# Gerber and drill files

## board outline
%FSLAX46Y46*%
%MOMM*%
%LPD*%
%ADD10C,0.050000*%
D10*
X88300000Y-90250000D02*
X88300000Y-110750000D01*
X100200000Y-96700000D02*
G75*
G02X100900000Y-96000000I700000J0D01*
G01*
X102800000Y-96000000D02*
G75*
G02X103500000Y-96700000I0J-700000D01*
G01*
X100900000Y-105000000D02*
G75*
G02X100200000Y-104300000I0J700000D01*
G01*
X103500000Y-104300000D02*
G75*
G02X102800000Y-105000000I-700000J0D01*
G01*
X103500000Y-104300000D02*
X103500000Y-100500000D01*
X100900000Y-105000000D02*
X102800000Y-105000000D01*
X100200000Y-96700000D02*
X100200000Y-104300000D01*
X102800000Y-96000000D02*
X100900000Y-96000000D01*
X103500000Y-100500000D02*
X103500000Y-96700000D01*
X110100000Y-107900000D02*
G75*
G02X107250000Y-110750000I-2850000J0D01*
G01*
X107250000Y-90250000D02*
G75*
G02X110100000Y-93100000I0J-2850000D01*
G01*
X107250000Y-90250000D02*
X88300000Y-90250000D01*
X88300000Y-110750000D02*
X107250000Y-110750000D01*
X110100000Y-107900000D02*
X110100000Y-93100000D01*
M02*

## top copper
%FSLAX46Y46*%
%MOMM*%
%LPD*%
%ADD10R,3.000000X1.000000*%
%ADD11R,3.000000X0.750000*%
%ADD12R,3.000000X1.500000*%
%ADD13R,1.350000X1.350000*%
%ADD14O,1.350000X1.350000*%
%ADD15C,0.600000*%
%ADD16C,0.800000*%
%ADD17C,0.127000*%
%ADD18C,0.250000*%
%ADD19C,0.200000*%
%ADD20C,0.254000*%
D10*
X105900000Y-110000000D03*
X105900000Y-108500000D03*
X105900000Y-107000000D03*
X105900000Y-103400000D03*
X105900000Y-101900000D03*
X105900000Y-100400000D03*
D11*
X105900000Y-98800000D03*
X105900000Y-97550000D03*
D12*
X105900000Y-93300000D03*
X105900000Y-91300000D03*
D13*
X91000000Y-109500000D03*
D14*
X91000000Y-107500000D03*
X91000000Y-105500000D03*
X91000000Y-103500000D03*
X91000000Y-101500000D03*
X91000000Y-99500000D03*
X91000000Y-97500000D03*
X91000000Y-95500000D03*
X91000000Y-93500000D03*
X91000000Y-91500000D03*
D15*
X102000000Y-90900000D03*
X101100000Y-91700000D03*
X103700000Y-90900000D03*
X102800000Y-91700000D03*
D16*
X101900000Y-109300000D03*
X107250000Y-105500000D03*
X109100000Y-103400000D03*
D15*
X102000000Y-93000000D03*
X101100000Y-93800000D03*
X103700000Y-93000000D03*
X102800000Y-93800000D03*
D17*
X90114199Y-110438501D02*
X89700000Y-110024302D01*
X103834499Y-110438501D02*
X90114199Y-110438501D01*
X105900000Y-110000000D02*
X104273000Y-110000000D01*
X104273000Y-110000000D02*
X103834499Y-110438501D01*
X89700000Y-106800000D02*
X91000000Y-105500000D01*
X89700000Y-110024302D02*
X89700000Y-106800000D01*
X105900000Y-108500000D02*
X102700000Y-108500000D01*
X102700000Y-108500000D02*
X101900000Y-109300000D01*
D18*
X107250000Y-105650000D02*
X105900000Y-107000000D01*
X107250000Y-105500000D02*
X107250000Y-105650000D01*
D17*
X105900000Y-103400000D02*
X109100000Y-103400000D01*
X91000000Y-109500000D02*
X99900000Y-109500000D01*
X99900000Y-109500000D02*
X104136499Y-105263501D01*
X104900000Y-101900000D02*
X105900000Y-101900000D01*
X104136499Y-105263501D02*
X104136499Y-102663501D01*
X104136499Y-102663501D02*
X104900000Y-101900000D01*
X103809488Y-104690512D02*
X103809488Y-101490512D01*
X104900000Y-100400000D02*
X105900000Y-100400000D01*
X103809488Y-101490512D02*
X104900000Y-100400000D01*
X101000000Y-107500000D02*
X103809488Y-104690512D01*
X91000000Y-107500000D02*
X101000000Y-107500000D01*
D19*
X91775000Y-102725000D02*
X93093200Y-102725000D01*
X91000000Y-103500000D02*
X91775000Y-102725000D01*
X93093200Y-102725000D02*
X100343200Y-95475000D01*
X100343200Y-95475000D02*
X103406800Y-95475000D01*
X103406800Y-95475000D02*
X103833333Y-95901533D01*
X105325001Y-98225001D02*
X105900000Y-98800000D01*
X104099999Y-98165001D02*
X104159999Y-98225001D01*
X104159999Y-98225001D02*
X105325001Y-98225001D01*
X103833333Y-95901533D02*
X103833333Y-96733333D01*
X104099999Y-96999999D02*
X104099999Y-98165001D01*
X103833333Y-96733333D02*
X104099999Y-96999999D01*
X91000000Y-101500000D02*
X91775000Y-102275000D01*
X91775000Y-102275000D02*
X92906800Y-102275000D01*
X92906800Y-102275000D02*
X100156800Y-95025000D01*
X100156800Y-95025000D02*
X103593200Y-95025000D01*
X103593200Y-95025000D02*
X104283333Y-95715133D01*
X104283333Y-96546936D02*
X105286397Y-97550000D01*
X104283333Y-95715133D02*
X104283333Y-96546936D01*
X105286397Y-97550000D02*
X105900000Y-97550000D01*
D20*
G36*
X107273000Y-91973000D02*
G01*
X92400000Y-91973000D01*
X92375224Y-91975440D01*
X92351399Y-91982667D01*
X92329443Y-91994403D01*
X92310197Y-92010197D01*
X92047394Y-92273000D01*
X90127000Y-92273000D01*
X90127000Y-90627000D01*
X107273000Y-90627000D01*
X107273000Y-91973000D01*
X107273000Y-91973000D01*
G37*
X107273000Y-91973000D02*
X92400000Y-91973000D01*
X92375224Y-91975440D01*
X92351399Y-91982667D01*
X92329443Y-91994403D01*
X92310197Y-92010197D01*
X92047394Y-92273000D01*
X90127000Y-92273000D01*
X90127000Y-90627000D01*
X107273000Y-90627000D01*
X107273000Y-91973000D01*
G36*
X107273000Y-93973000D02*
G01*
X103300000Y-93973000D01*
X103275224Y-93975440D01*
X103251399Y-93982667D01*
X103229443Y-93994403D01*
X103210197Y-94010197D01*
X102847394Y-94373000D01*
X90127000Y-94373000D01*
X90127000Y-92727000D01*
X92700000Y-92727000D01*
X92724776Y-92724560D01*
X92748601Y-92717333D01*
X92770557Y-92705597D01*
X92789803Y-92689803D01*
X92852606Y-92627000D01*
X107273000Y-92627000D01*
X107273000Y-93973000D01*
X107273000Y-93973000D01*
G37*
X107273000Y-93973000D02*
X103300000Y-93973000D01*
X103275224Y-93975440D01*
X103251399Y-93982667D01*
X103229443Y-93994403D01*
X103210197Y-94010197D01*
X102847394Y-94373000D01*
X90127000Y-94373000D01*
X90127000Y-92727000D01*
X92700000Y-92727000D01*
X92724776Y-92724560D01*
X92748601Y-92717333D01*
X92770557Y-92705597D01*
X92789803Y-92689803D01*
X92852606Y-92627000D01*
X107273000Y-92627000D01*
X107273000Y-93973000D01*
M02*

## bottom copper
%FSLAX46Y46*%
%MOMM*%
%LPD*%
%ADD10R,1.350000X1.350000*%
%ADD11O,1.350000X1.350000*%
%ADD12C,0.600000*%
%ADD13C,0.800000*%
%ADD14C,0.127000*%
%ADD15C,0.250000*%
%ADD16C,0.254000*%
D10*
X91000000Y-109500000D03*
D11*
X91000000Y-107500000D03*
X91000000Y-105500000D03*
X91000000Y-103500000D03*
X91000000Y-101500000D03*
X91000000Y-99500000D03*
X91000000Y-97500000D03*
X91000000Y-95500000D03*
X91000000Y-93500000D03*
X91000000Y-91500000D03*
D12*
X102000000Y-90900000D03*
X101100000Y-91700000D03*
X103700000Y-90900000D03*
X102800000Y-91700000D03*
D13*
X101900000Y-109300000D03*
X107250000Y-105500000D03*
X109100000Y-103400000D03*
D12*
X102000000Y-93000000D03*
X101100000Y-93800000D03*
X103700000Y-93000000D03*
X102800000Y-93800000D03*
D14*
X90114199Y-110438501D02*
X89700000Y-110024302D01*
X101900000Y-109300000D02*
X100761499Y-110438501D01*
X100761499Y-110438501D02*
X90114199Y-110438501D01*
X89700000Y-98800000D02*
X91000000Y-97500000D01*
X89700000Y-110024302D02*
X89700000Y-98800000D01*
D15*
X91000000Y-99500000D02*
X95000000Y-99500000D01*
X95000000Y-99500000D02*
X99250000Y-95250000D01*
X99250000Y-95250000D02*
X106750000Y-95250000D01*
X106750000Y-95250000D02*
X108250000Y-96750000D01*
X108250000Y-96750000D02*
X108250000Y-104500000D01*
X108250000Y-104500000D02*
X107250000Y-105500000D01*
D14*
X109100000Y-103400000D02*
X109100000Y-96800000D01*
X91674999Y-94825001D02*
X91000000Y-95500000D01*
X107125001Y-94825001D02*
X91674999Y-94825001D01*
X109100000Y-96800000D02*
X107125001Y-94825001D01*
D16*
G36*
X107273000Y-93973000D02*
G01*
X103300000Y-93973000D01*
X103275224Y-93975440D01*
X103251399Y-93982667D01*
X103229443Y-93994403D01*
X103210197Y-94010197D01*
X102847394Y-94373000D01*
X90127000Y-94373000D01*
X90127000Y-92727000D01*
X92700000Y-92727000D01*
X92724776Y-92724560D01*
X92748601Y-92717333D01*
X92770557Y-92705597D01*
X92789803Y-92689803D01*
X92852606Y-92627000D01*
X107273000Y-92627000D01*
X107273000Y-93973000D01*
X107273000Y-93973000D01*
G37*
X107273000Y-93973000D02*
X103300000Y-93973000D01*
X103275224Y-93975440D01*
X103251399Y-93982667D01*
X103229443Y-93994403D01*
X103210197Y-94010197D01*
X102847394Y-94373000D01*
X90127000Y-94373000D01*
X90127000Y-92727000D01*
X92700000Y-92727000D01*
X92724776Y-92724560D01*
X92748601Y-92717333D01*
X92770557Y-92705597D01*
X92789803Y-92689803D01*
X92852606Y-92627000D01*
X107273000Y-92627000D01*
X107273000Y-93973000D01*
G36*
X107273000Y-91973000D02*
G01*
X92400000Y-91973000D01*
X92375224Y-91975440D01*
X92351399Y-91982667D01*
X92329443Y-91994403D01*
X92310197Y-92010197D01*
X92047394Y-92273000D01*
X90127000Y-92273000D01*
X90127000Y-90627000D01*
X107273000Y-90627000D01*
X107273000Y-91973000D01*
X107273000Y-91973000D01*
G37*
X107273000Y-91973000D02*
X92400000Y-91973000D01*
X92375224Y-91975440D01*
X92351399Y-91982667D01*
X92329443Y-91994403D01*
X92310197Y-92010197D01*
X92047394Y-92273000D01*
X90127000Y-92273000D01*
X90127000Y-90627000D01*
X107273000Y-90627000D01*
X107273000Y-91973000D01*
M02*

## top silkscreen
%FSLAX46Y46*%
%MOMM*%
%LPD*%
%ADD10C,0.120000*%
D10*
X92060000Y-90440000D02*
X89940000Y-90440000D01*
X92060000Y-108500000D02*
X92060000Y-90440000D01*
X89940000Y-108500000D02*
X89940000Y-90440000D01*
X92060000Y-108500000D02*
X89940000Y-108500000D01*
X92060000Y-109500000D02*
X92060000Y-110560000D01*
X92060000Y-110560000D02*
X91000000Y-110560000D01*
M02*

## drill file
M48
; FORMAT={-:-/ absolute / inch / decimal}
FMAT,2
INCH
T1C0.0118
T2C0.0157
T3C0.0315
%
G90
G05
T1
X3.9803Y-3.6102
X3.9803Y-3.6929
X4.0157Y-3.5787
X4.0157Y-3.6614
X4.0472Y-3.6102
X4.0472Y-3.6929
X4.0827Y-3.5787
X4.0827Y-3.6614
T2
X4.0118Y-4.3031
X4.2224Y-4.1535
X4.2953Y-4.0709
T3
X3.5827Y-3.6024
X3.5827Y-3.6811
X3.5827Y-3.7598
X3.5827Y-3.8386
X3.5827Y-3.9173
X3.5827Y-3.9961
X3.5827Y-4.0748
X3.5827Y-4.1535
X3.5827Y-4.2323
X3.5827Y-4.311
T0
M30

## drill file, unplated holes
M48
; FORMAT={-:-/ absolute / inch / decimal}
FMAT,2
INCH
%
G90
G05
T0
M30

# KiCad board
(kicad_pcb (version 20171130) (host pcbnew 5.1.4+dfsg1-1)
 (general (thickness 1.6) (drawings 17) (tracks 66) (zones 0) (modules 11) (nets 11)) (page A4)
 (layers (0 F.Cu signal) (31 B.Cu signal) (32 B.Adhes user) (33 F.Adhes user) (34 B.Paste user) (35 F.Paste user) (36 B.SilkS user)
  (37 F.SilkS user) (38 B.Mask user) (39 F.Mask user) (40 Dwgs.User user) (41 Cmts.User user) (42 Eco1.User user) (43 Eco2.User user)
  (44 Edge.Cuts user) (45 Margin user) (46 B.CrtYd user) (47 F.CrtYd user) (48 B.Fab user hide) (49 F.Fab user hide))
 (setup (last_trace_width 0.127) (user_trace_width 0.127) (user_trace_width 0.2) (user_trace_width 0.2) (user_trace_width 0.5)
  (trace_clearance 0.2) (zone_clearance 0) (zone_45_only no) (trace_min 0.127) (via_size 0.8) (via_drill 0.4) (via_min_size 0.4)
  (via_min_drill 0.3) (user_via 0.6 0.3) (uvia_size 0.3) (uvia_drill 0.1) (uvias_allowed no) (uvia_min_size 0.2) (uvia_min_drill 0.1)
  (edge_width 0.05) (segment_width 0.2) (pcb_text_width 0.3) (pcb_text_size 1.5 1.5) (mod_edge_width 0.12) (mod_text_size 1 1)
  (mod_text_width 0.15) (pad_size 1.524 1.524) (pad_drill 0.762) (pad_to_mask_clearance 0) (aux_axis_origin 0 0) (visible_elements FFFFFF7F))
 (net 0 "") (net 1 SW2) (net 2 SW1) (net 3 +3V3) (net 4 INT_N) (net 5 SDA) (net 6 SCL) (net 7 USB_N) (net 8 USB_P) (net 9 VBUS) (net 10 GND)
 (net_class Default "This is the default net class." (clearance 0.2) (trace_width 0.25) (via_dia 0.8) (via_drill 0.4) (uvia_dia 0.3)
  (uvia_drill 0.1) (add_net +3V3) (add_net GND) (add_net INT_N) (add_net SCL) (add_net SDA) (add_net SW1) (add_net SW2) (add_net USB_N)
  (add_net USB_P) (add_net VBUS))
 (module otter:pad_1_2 (layer F.Cu) (at 105.9 110 90)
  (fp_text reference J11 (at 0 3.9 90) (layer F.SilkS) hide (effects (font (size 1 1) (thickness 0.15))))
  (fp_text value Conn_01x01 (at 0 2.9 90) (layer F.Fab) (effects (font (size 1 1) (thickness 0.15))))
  (pad 1 smd rect (at 0 0 90) (size 1 3) (layers F.Cu F.Paste F.Mask) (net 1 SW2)))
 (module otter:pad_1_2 (layer F.Cu) (at 105.9 108.5 90)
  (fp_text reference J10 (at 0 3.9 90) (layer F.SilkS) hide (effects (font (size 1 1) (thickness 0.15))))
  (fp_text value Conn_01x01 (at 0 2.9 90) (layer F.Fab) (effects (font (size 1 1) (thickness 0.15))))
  (pad 1 smd rect (at 0 0 90) (size 1 3) (layers F.Cu F.Paste F.Mask) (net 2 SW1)))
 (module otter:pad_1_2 (layer F.Cu) (at 105.9 107 90)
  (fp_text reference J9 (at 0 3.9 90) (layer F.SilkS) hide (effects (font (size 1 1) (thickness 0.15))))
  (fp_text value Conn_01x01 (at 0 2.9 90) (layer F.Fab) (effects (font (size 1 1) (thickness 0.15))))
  (pad 1 smd rect (at 0 0 90) (size 1 3) (layers F.Cu F.Paste F.Mask) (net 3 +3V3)))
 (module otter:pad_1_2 (layer F.Cu) (at 105.9 103.4 90)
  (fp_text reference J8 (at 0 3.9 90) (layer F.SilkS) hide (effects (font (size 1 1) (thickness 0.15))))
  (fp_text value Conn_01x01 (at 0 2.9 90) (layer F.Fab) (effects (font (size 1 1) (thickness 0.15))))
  (pad 1 smd rect (at 0 0 90) (size 1 3) (layers F.Cu F.Paste F.Mask) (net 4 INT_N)))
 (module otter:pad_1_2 (layer F.Cu) (at 105.9 101.9 90)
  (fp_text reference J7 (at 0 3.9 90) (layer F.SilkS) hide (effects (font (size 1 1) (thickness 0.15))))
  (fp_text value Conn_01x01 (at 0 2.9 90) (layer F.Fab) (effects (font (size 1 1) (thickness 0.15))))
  (pad 1 smd rect (at 0 0 90) (size 1 3) (layers F.Cu F.Paste F.Mask) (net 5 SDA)))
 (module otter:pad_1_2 (layer F.Cu) (at 105.9 100.4 90)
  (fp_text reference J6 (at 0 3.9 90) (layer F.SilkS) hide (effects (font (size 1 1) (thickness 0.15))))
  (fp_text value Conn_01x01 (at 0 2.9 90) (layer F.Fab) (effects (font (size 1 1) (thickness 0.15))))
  (pad 1 smd rect (at 0 0 90) (size 1 3) (layers F.Cu F.Paste F.Mask) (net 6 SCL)))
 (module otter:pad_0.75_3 (layer F.Cu) (at 105.9 98.8 90)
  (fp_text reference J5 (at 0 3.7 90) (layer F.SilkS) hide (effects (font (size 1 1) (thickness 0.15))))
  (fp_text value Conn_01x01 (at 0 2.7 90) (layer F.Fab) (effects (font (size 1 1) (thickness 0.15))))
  (pad 1 smd rect (at 0 0 90) (size 0.75 3) (layers F.Cu F.Paste F.Mask) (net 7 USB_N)))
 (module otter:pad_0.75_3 (layer F.Cu) (at 105.9 97.55 90)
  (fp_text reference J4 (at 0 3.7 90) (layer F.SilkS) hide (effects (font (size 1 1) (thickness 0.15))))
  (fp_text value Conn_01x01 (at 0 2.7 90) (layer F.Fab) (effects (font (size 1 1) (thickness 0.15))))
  (pad 1 smd rect (at 0 0 90) (size 0.75 3) (layers F.Cu F.Paste F.Mask) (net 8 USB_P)))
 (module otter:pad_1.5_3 (layer F.Cu) (at 105.9 93.3 90)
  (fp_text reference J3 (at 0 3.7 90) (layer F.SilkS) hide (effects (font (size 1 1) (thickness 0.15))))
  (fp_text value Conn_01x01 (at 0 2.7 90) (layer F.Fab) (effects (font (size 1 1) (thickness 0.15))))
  (pad 1 smd rect (at 0 0 90) (size 1.5 3) (layers F.Cu F.Paste F.Mask) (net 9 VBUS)))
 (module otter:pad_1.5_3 (layer F.Cu) (at 105.9 91.3 90)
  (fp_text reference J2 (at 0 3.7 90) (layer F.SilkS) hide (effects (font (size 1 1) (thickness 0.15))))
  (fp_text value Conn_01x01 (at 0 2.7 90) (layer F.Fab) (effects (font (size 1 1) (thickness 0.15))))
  (pad 1 smd rect (at 0 0 90) (size 1.5 3) (layers F.Cu F.Paste F.Mask) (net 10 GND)))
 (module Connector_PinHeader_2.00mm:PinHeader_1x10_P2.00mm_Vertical (layer F.Cu) (at 91 100.5 180)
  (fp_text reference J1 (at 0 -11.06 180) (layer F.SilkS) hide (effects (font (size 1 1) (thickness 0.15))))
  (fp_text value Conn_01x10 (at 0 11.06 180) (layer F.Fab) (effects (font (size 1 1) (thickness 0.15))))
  (fp_line (start -1.06 10.06) (end 1.06 10.06) (layer F.SilkS) (width 0.12))
  (fp_line (start -1.06 -8) (end -1.06 10.06) (layer F.SilkS) (width 0.12))
  (fp_line (start 1.06 -8) (end 1.06 10.06) (layer F.SilkS) (width 0.12))
  (fp_line (start -1.06 -8) (end 1.06 -8) (layer F.SilkS) (width 0.12))
  (fp_line (start -1.06 -9) (end -1.06 -10.06) (layer F.SilkS) (width 0.12))
  (fp_line (start -1.06 -10.06) (end 0 -10.06) (layer F.SilkS) (width 0.12))
  (pad 1 thru_hole rect (at 0 -9 180) (size 1.35 1.35) (drill 0.8) (layers *.Cu *.Mask) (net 5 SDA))
  (pad 2 thru_hole oval (at 0 -7 180) (size 1.35 1.35) (drill 0.8) (layers *.Cu *.Mask) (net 6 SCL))
  (pad 3 thru_hole oval (at 0 -5 180) (size 1.35 1.35) (drill 0.8) (layers *.Cu *.Mask) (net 1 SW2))
  (pad 4 thru_hole oval (at 0 -3 180) (size 1.35 1.35) (drill 0.8) (layers *.Cu *.Mask) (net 7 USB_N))
  (pad 5 thru_hole oval (at 0 -1 180) (size 1.35 1.35) (drill 0.8) (layers *.Cu *.Mask) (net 8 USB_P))
  (pad 6 thru_hole oval (at 0 1 180) (size 1.35 1.35) (drill 0.8) (layers *.Cu *.Mask) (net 3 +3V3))
  (pad 7 thru_hole oval (at 0 3 180) (size 1.35 1.35) (drill 0.8) (layers *.Cu *.Mask) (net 2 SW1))
  (pad 8 thru_hole oval (at 0 5 180) (size 1.35 1.35) (drill 0.8) (layers *.Cu *.Mask) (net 4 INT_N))
  (pad 9 thru_hole oval (at 0 7 180) (size 1.35 1.35) (drill 0.8) (layers *.Cu *.Mask) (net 9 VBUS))
  (pad 10 thru_hole oval (at 0 9 180) (size 1.35 1.35) (drill 0.8) (layers *.Cu *.Mask) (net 10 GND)))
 (gr_line (start 88.3 90.25) (end 88.3 110.75) (layer Edge.Cuts) (width 0.05))
 (gr_arc (start 100.9 96.7) (end 100.9 96) (angle -90) (layer Edge.Cuts) (width 0.05))
 (gr_arc (start 102.8 96.7) (end 103.5 96.7) (angle -90) (layer Edge.Cuts) (width 0.05))
 (gr_arc (start 100.9 104.3) (end 100.2 104.3) (angle -90) (layer Edge.Cuts) (width 0.05))
 (gr_arc (start 102.8 104.3) (end 102.8 105) (angle -90) (layer Edge.Cuts) (width 0.05))
 (gr_line (start 103.5 104.3) (end 103.5 100.5) (layer Edge.Cuts) (width 0.05))
 (gr_line (start 100.9 105) (end 102.8 105) (layer Edge.Cuts) (width 0.05))
 (gr_line (start 100.2 96.7) (end 100.2 104.3) (layer Edge.Cuts) (width 0.05))
 (gr_line (start 102.8 96) (end 100.9 96) (layer Edge.Cuts) (width 0.05))
 (gr_line (start 103.5 100.5) (end 103.5 96.7) (layer Edge.Cuts) (width 0.05))
 (gr_arc (start 107.25 107.9) (end 107.25 110.75) (angle -90) (layer Edge.Cuts) (width 0.05))
 (gr_arc (start 107.25 93.1) (end 110.1 93.1) (angle -90) (layer Edge.Cuts) (width 0.05))
 (gr_line (start 107.25 90.25) (end 88.3 90.25) (layer Edge.Cuts) (width 0.05))
 (gr_line (start 88.3 110.75) (end 107.25 110.75) (layer Edge.Cuts) (width 0.05))
 (gr_line (start 110.1 107.9) (end 110.1 93.1) (layer Edge.Cuts) (width 0.05))
 (via (at 102 90.9) (size 0.6) (drill 0.3) (layers F.Cu B.Cu) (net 10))
 (via (at 101.1 91.7) (size 0.6) (drill 0.3) (layers F.Cu B.Cu) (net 10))
 (via (at 103.7 90.9) (size 0.6) (drill 0.3) (layers F.Cu B.Cu) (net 10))
 (via (at 102.8 91.7) (size 0.6) (drill 0.3) (layers F.Cu B.Cu) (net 10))
 (segment (start 90.114199 110.438501) (end 89.7 110.024302) (width 0.127) (layer F.Cu) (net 1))
 (segment (start 103.834499 110.438501) (end 90.114199 110.438501) (width 0.127) (layer F.Cu) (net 1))
 (segment (start 105.9 110) (end 104.273 110) (width 0.127) (layer F.Cu) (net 1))
 (segment (start 104.273 110) (end 103.834499 110.438501) (width 0.127) (layer F.Cu) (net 1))
 (segment (start 89.7 106.8) (end 91 105.5) (width 0.127) (layer F.Cu) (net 1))
 (segment (start 89.7 110.024302) (end 89.7 106.8) (width 0.127) (layer F.Cu) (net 1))
 (via (at 101.9 109.3) (size 0.8) (drill 0.4) (layers F.Cu B.Cu) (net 2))
 (segment (start 105.9 108.5) (end 102.7 108.5) (width 0.127) (layer F.Cu) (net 2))
 (segment (start 102.7 108.5) (end 101.9 109.3) (width 0.127) (layer F.Cu) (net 2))
 (segment (start 90.114199 110.438501) (end 89.7 110.024302) (width 0.127) (layer B.Cu) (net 2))
 (segment (start 101.9 109.3) (end 100.761499 110.438501) (width 0.127) (layer B.Cu) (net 2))
 (segment (start 100.761499 110.438501) (end 90.114199 110.438501) (width 0.127) (layer B.Cu) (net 2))
 (segment (start 89.7 98.8) (end 91 97.5) (width 0.127) (layer B.Cu) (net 2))
 (segment (start 89.7 110.024302) (end 89.7 98.8) (width 0.127) (layer B.Cu) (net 2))
 (segment (start 91 99.5) (end 95 99.5) (width 0.25) (layer B.Cu) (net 3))
 (segment (start 95 99.5) (end 99.25 95.25) (width 0.25) (layer B.Cu) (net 3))
 (segment (start 99.25 95.25) (end 106.75 95.25) (width 0.25) (layer B.Cu) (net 3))
 (segment (start 106.75 95.25) (end 108.25 96.75) (width 0.25) (layer B.Cu) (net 3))
 (segment (start 108.25 96.75) (end 108.25 104.5) (width 0.25) (layer B.Cu) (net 3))
 (via (at 107.25 105.5) (size 0.8) (drill 0.4) (layers F.Cu B.Cu) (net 3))
 (segment (start 108.25 104.5) (end 107.25 105.5) (width 0.25) (layer B.Cu) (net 3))
 (segment (start 107.25 105.65) (end 105.9 107) (width 0.25) (layer F.Cu) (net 3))
 (segment (start 107.25 105.5) (end 107.25 105.65) (width 0.25) (layer F.Cu) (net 3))
 (via (at 109.1 103.4) (size 0.8) (drill 0.4) (layers F.Cu B.Cu) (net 4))
 (segment (start 105.9 103.4) (end 109.1 103.4) (width 0.127) (layer F.Cu) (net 4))
 (segment (start 109.1 103.4) (end 109.1 96.8) (width 0.127) (layer B.Cu) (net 4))
 (segment (start 91.674999 94.825001) (end 91 95.5) (width 0.127) (layer B.Cu) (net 4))
 (segment (start 107.125001 94.825001) (end 91.674999 94.825001) (width 0.127) (layer B.Cu) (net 4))
 (segment (start 109.1 96.8) (end 107.125001 94.825001) (width 0.127) (layer B.Cu) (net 4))
 (segment (start 91 109.5) (end 99.9 109.5) (width 0.127) (layer F.Cu) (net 5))
 (segment (start 99.9 109.5) (end 104.136499 105.263501) (width 0.127) (layer F.Cu) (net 5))
 (segment (start 104.9 101.9) (end 105.9 101.9) (width 0.127) (layer F.Cu) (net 5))
 (segment (start 104.136499 105.263501) (end 104.136499 102.663501) (width 0.127) (layer F.Cu) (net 5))
 (segment (start 104.136499 102.663501) (end 104.9 101.9) (width 0.127) (layer F.Cu) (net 5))
 (segment (start 103.809488 104.690512) (end 103.809488 101.490512) (width 0.127) (layer F.Cu) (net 6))
 (segment (start 104.9 100.4) (end 105.9 100.4) (width 0.127) (layer F.Cu) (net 6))
 (segment (start 103.809488 101.490512) (end 104.9 100.4) (width 0.127) (layer F.Cu) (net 6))
 (segment (start 101 107.5) (end 103.809488 104.690512) (width 0.127) (layer F.Cu) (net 6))
 (segment (start 91 107.5) (end 101 107.5) (width 0.127) (layer F.Cu) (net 6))
 (segment (start 91.775 102.725) (end 93.0932 102.725) (width 0.2) (layer F.Cu) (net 7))
 (segment (start 91 103.5) (end 91.775 102.725) (width 0.2) (layer F.Cu) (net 7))
 (segment (start 93.0932 102.725) (end 100.3432 95.475) (width 0.2) (layer F.Cu) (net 7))
 (segment (start 100.3432 95.475) (end 103.4068 95.475) (width 0.2) (layer F.Cu) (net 7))
 (segment (start 103.4068 95.475) (end 103.833333 95.901533) (width 0.2) (layer F.Cu) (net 7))
 (segment (start 105.325001 98.225001) (end 105.9 98.8) (width 0.2) (layer F.Cu) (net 7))
 (segment (start 104.099999 98.165001) (end 104.159999 98.225001) (width 0.2) (layer F.Cu) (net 7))
 (segment (start 104.159999 98.225001) (end 105.325001 98.225001) (width 0.2) (layer F.Cu) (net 7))
 (segment (start 103.833333 95.901533) (end 103.833333 96.733333) (width 0.2) (layer F.Cu) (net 7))
 (segment (start 104.099999 96.999999) (end 104.099999 98.165001) (width 0.2) (layer F.Cu) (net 7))
 (segment (start 103.833333 96.733333) (end 104.099999 96.999999) (width 0.2) (layer F.Cu) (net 7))
 (segment (start 91 101.5) (end 91.775 102.275) (width 0.2) (layer F.Cu) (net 8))
 (segment (start 91.775 102.275) (end 92.9068 102.275) (width 0.2) (layer F.Cu) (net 8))
 (segment (start 92.9068 102.275) (end 100.1568 95.025) (width 0.2) (layer F.Cu) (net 8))
 (segment (start 100.1568 95.025) (end 103.5932 95.025) (width 0.2) (layer F.Cu) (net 8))
 (segment (start 103.5932 95.025) (end 104.283333 95.715133) (width 0.2) (layer F.Cu) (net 8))
 (segment (start 104.283333 96.546936) (end 105.286397 97.55) (width 0.2) (layer F.Cu) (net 8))
 (segment (start 104.283333 95.715133) (end 104.283333 96.546936) (width 0.2) (layer F.Cu) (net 8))
 (segment (start 105.286397 97.55) (end 105.9 97.55) (width 0.2) (layer F.Cu) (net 8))
 (via (at 102 93) (size 0.6) (drill 0.3) (layers F.Cu B.Cu) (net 9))
 (via (at 101.1 93.8) (size 0.6) (drill 0.3) (layers F.Cu B.Cu) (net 9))
 (via (at 103.7 93) (size 0.6) (drill 0.3) (layers F.Cu B.Cu) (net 9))
 (via (at 102.8 93.8) (size 0.6) (drill 0.3) (layers F.Cu B.Cu) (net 9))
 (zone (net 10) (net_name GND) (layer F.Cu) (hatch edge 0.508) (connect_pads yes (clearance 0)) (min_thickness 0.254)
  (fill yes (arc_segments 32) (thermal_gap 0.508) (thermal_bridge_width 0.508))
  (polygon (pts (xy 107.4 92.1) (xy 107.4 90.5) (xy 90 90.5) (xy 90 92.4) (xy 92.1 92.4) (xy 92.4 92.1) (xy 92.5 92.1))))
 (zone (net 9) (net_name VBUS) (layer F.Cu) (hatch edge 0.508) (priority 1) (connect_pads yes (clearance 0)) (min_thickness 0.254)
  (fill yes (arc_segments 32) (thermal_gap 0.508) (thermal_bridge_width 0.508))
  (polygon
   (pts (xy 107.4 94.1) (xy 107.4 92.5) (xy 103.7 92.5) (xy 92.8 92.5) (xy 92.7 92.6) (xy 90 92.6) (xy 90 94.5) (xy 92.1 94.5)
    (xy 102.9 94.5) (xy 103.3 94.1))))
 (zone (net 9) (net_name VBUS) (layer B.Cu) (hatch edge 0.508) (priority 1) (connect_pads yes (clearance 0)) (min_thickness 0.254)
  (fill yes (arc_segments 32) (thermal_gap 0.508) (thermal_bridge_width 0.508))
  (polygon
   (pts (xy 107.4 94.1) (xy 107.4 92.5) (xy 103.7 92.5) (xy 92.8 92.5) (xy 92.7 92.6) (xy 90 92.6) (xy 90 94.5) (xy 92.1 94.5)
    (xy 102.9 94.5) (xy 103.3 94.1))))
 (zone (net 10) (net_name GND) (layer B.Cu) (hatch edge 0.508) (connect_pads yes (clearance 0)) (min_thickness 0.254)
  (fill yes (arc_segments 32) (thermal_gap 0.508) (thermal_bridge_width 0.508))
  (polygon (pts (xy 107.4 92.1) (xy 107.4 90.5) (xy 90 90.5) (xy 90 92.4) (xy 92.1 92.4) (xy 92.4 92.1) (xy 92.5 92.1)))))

